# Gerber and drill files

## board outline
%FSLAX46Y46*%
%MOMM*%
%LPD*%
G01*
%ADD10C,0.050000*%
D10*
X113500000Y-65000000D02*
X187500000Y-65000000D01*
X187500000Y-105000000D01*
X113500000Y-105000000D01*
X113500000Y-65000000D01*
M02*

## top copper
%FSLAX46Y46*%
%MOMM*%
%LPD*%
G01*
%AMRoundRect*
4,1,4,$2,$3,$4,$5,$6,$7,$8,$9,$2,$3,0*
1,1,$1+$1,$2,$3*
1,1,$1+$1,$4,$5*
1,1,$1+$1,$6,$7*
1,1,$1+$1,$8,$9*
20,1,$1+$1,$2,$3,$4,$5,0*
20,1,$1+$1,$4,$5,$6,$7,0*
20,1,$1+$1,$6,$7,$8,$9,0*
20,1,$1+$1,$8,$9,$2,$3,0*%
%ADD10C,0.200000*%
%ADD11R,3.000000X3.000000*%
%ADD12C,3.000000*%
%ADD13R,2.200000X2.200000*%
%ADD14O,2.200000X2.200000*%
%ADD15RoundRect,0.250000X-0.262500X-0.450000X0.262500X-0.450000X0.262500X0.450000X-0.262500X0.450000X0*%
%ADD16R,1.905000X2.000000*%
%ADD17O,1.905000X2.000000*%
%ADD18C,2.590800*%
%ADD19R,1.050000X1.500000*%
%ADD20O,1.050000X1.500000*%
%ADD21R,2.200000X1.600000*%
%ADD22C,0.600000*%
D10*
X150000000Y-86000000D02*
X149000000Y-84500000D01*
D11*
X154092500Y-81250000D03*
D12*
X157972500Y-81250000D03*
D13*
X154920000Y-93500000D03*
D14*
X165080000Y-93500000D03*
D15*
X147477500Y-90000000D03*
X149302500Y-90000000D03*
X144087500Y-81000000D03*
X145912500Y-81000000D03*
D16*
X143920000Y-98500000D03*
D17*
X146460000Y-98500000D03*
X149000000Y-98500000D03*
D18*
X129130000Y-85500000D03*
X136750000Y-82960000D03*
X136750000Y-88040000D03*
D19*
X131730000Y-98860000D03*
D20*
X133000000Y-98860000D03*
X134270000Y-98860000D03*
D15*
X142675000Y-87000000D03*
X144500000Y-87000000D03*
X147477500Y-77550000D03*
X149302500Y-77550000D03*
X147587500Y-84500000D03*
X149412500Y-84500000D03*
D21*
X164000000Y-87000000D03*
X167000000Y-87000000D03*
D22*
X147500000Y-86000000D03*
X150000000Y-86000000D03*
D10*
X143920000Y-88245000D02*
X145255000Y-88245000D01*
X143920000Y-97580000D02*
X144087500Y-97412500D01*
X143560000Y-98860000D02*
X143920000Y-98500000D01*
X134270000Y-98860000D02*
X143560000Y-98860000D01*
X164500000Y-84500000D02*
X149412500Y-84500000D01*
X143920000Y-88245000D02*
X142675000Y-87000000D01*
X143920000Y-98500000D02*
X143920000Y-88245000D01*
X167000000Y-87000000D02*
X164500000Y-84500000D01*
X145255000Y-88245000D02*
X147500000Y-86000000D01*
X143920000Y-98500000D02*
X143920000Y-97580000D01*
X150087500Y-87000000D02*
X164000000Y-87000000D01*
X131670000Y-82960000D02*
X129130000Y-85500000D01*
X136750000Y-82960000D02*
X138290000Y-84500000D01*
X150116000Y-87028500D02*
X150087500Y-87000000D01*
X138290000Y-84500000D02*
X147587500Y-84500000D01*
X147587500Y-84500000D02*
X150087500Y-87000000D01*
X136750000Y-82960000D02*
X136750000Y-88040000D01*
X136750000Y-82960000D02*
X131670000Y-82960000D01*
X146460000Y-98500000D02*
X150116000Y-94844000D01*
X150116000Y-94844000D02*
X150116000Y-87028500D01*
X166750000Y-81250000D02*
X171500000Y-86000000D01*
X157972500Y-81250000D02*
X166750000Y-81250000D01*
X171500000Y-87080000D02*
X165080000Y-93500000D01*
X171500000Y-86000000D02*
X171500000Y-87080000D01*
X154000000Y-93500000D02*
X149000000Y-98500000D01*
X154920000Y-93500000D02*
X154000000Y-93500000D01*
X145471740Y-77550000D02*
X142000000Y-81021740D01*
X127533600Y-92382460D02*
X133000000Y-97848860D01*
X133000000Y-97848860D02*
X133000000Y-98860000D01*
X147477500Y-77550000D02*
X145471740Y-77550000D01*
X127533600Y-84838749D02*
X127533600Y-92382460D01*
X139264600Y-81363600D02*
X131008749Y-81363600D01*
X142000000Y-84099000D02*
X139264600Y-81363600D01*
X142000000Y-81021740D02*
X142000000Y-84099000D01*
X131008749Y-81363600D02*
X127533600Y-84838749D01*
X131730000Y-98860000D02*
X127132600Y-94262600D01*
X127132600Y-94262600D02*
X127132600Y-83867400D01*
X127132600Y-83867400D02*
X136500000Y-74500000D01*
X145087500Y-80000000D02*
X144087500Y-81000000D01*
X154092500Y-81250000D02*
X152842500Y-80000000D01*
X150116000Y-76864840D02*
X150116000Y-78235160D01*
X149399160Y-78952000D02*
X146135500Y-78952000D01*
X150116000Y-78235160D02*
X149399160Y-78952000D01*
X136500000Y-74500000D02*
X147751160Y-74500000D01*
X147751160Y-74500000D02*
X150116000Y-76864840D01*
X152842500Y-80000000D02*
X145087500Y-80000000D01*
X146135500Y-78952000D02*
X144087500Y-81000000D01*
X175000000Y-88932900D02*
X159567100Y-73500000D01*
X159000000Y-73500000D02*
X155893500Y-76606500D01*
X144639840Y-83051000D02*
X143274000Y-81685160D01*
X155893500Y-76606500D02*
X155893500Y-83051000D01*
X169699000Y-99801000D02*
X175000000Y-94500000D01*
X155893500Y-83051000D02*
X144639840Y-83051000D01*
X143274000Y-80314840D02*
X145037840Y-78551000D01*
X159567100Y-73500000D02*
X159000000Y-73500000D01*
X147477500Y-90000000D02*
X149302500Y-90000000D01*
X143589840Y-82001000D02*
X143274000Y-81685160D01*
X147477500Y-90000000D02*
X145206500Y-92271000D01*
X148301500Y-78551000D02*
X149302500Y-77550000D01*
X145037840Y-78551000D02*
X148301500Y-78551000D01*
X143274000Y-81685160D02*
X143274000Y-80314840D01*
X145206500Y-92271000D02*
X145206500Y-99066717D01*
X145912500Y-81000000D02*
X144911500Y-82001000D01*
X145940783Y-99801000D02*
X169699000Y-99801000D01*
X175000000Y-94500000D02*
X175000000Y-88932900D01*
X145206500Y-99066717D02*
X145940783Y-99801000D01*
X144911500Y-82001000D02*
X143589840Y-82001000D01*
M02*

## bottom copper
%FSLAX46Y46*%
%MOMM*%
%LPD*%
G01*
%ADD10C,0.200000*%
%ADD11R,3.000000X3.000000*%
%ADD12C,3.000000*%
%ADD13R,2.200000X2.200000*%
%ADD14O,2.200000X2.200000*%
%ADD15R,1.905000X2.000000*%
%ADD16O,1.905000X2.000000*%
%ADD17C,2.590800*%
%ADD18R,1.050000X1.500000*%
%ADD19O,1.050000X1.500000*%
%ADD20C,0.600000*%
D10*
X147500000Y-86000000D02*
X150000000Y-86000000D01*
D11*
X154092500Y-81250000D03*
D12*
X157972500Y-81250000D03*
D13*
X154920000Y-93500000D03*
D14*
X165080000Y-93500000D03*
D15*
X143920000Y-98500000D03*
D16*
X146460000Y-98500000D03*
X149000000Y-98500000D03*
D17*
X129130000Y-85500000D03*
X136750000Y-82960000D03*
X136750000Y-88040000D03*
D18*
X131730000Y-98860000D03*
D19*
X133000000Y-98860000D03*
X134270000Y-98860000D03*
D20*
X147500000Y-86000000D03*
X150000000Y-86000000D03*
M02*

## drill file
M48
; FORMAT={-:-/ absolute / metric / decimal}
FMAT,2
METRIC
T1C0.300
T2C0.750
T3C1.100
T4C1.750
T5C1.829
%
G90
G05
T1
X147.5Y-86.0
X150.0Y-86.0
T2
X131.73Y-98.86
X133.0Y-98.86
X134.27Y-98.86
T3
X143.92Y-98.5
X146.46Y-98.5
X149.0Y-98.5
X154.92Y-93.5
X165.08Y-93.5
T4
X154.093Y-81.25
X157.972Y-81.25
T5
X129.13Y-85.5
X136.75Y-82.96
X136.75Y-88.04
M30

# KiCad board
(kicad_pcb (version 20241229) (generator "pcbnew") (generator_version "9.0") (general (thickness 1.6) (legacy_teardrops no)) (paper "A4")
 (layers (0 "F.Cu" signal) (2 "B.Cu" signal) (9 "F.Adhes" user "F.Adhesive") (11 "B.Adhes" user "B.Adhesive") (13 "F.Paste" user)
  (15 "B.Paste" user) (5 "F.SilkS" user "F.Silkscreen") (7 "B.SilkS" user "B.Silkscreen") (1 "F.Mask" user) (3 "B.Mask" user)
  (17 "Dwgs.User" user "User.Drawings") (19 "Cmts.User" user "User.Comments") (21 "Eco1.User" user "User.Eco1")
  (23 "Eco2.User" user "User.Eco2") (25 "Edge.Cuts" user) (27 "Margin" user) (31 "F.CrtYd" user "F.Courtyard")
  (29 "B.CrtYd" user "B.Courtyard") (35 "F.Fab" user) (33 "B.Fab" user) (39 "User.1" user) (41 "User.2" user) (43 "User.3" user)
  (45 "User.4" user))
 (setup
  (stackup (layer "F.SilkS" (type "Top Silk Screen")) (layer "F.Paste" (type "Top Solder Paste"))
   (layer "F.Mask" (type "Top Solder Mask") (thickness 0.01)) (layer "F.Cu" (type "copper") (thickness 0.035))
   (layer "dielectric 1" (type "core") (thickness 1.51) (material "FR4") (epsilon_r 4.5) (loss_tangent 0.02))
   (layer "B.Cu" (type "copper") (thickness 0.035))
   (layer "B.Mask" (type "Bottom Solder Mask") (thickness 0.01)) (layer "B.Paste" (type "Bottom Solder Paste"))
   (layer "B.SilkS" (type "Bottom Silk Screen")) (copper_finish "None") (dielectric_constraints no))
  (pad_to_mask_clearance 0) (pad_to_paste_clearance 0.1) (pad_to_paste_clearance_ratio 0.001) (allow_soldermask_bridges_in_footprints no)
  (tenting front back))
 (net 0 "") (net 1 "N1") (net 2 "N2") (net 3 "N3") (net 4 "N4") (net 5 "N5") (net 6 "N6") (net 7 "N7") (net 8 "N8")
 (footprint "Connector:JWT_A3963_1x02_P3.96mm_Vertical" (layer "F.Cu") (at 154.0925 81.25)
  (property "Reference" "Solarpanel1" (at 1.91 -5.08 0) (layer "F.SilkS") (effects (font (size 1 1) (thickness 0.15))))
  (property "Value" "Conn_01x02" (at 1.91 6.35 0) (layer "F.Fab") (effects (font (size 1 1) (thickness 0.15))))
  (pad "1" thru_hole rect (at 0 0) (size 3 3) (drill 1.75) (layers "*.Cu" "*.Mask") (remove_unused_layers no) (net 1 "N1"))
  (pad "2" thru_hole circle (at 3.88 0) (size 3 3) (drill 1.75) (layers "*.Cu" "*.Mask") (remove_unused_layers no) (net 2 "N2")))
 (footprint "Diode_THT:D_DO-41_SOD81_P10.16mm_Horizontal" (layer "F.Cu") (at 154.92 93.5)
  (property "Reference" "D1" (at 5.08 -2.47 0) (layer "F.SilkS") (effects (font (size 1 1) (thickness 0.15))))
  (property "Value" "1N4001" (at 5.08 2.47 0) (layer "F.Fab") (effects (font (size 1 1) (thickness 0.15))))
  (pad "1" thru_hole rect (at 0 0) (size 2.2 2.2) (drill 1.1) (layers "*.Cu" "*.Mask") (remove_unused_layers no) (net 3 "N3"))
  (pad "2" thru_hole oval (at 10.16 0) (size 2.2 2.2) (drill 1.1) (layers "*.Cu" "*.Mask") (remove_unused_layers no) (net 2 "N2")))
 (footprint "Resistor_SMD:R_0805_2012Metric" (layer "F.Cu") (at 148.39 90)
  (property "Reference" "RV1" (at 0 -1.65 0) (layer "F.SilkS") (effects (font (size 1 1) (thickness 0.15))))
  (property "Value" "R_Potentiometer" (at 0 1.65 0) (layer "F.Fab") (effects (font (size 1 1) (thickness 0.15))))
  (pad "1" smd roundrect (at -0.9125 0) (size 1.025 1.4) (layers "F.Cu" "F.Mask" "F.Paste") (roundrect_rratio 0.243902) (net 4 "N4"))
  (pad "2" smd roundrect (at 0.9125 0) (size 1.025 1.4) (layers "F.Cu" "F.Mask" "F.Paste") (roundrect_rratio 0.243902) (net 4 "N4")))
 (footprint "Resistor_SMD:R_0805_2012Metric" (layer "F.Cu") (at 145 81)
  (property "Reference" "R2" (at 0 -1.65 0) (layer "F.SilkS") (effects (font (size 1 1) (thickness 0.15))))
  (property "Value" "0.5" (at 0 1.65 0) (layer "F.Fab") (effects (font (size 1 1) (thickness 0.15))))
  (pad "1" smd roundrect (at -0.9125 0) (size 1.025 1.4) (layers "F.Cu" "F.Mask" "F.Paste") (roundrect_rratio 0.243902) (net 1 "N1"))
  (pad "2" smd roundrect (at 0.9125 0) (size 1.025 1.4) (layers "F.Cu" "F.Mask" "F.Paste") (roundrect_rratio 0.243902) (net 4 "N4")))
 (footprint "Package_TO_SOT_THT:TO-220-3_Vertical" (layer "F.Cu") (at 143.92 98.5)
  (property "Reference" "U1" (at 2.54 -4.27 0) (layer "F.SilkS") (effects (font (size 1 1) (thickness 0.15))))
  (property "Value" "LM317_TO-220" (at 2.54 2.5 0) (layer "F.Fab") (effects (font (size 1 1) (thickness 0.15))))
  (pad "1" thru_hole rect (at 0 0) (size 1.905 2) (drill 1.1) (layers "*.Cu" "*.Mask") (remove_unused_layers no) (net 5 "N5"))
  (pad "2" thru_hole oval (at 2.54 0) (size 1.905 2) (drill 1.1) (layers "*.Cu" "*.Mask") (remove_unused_layers no) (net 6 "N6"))
  (pad "3" thru_hole oval (at 5.08 0) (size 1.905 2) (drill 1.1) (layers "*.Cu" "*.Mask") (remove_unused_layers no) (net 3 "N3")))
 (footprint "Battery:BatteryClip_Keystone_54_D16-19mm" (layer "F.Cu") (at 129.13 85.5)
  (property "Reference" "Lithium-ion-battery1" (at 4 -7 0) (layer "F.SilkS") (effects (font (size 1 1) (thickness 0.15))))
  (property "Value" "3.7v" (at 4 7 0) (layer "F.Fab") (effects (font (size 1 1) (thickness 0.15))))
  (pad "1" thru_hole circle (at 0 0 180) (size 2.5908 2.5908) (drill 1.8288) (layers "*.Cu" "*.Mask") (remove_unused_layers no) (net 6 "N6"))
  (pad "1" thru_hole circle (at 7.62 -2.54 180) (size 2.5908 2.5908) (drill 1.8288) (layers "*.Cu" "*.Mask") (remove_unused_layers no)
   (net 6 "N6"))
  (pad "1" thru_hole circle (at 7.62 2.54 180) (size 2.5908 2.5908) (drill 1.8288) (layers "*.Cu" "*.Mask") (remove_unused_layers no)
   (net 6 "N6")))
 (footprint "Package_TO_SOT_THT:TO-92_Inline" (layer "F.Cu") (at 131.73 98.86)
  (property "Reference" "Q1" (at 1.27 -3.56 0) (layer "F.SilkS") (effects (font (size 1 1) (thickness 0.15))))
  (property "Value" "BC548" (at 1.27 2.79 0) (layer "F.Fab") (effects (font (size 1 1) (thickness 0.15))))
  (pad "1" thru_hole rect (at 0 0) (size 1.05 1.5) (drill 0.75) (layers "*.Cu" "*.Mask") (remove_unused_layers no) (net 1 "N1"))
  (pad "2" thru_hole oval (at 1.27 0) (size 1.05 1.5) (drill 0.75) (layers "*.Cu" "*.Mask") (remove_unused_layers no) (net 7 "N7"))
  (pad "3" thru_hole oval (at 2.54 0) (size 1.05 1.5) (drill 0.75) (layers "*.Cu" "*.Mask") (remove_unused_layers no) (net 5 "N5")))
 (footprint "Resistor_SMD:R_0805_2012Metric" (layer "F.Cu") (at 143.5875 87)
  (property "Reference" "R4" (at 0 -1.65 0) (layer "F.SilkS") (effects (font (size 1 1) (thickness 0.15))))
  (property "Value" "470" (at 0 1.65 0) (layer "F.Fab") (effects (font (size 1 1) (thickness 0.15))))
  (pad "1" smd roundrect (at -0.9125 0) (size 1.025 1.4) (layers "F.Cu" "F.Mask" "F.Paste") (roundrect_rratio 0.243902) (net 5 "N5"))
  (pad "2" smd roundrect (at 0.9125 0) (size 1.025 1.4) (layers "F.Cu" "F.Mask" "F.Paste") (roundrect_rratio 0.243902) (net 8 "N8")))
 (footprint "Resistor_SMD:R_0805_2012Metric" (layer "F.Cu") (at 148.39 77.55)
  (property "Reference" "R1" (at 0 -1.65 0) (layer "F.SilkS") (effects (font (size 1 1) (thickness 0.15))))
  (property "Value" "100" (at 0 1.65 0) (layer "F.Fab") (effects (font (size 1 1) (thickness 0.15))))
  (pad "1" smd roundrect (at -0.9125 0) (size 1.025 1.4) (layers "F.Cu" "F.Mask" "F.Paste") (roundrect_rratio 0.243902) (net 7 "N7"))
  (pad "2" smd roundrect (at 0.9125 0) (size 1.025 1.4) (layers "F.Cu" "F.Mask" "F.Paste") (roundrect_rratio 0.243902) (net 4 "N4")))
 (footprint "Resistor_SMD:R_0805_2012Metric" (layer "F.Cu") (at 148.5 84.5)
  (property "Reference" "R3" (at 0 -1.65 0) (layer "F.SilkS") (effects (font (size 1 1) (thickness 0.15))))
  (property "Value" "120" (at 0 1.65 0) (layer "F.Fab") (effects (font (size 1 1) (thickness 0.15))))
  (pad "1" smd roundrect (at -0.9125 0) (size 1.025 1.4) (layers "F.Cu" "F.Mask" "F.Paste") (roundrect_rratio 0.243902) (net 6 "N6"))
  (pad "2" smd roundrect (at 0.9125 0) (size 1.025 1.4) (layers "F.Cu" "F.Mask" "F.Paste") (roundrect_rratio 0.243902) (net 5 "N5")))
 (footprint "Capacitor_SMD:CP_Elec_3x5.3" (layer "F.Cu") (at 165.5 87)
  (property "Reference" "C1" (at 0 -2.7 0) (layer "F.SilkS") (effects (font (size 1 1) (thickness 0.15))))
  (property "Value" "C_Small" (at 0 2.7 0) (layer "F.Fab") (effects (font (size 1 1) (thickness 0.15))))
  (pad "1" smd rect (at -1.5 0) (size 2.2 1.6) (layers "F.Cu" "F.Mask" "F.Paste") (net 6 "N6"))
  (pad "2" smd rect (at 1.5 0) (size 2.2 1.6) (layers "F.Cu" "F.Mask" "F.Paste") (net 5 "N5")))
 (gr_line (start 150 86) (end 149 84.5) (stroke (width 0.2) (type default)) (layer "F.Cu") (net 5))
 (gr_line (start 147.5 86) (end 150 86) (stroke (width 0.2) (type default)) (layer "B.Cu") (net 5))
 (gr_rect (start 113.5 65) (end 187.5 105) (stroke (width 0.05) (type default)) (fill no) (layer "Edge.Cuts"))
 (segment (start 143.92 88.245) (end 145.255 88.245) (width 0.2) (layer "F.Cu") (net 5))
 (segment (start 143.92 97.58) (end 144.0875 97.4125) (width 0.2) (layer "F.Cu") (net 5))
 (segment (start 143.56 98.86) (end 143.92 98.5) (width 0.2) (layer "F.Cu") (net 5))
 (segment (start 134.27 98.86) (end 143.56 98.86) (width 0.2) (layer "F.Cu") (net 5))
 (segment (start 164.5 84.5) (end 149.4125 84.5) (width 0.2) (layer "F.Cu") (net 5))
 (segment (start 143.92 88.245) (end 142.675 87) (width 0.2) (layer "F.Cu") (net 5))
 (segment (start 143.92 98.5) (end 143.92 88.245) (width 0.2) (layer "F.Cu") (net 5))
 (segment (start 167 87) (end 164.5 84.5) (width 0.2) (layer "F.Cu") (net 5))
 (segment (start 145.255 88.245) (end 147.5 86) (width 0.2) (layer "F.Cu") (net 5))
 (segment (start 143.92 98.5) (end 143.92 97.58) (width 0.2) (layer "F.Cu") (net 5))
 (via (at 147.5 86) (size 0.6) (drill 0.3) (layers "F.Cu" "B.Cu") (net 5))
 (via (at 150 86) (size 0.6) (drill 0.3) (layers "F.Cu" "B.Cu") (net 5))
 (segment (start 150.0875 87) (end 164 87) (width 0.2) (layer "F.Cu") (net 6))
 (segment (start 131.67 82.96) (end 129.13 85.5) (width 0.2) (layer "F.Cu") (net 6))
 (segment (start 136.75 82.96) (end 138.29 84.5) (width 0.2) (layer "F.Cu") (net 6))
 (segment (start 150.116 87.0285) (end 150.0875 87) (width 0.2) (layer "F.Cu") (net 6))
 (segment (start 138.29 84.5) (end 147.5875 84.5) (width 0.2) (layer "F.Cu") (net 6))
 (segment (start 147.5875 84.5) (end 150.0875 87) (width 0.2) (layer "F.Cu") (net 6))
 (segment (start 136.75 82.96) (end 136.75 88.04) (width 0.2) (layer "F.Cu") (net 6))
 (segment (start 136.75 82.96) (end 131.67 82.96) (width 0.2) (layer "F.Cu") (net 6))
 (segment (start 146.46 98.5) (end 150.116 94.844) (width 0.2) (layer "F.Cu") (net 6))
 (segment (start 150.116 94.844) (end 150.116 87.0285) (width 0.2) (layer "F.Cu") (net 6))
 (segment (start 166.75 81.25) (end 171.5 86) (width 0.2) (layer "F.Cu") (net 2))
 (segment (start 157.9725 81.25) (end 166.75 81.25) (width 0.2) (layer "F.Cu") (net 2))
 (segment (start 171.5 87.08) (end 165.08 93.5) (width 0.2) (layer "F.Cu") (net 2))
 (segment (start 171.5 86) (end 171.5 87.08) (width 0.2) (layer "F.Cu") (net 2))
 (segment (start 154 93.5) (end 149 98.5) (width 0.2) (layer "F.Cu") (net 3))
 (segment (start 154.92 93.5) (end 154 93.5) (width 0.2) (layer "F.Cu") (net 3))
 (segment (start 145.47174 77.55) (end 142 81.02174) (width 0.2) (layer "F.Cu") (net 7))
 (segment (start 127.5336 92.38246) (end 133 97.84886) (width 0.2) (layer "F.Cu") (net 7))
 (segment (start 133 97.84886) (end 133 98.86) (width 0.2) (layer "F.Cu") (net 7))
 (segment (start 147.4775 77.55) (end 145.47174 77.55) (width 0.2) (layer "F.Cu") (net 7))
 (segment (start 127.5336 84.838749) (end 127.5336 92.38246) (width 0.2) (layer "F.Cu") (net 7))
 (segment (start 139.2646 81.3636) (end 131.008749 81.3636) (width 0.2) (layer "F.Cu") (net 7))
 (segment (start 142 84.099) (end 139.2646 81.3636) (width 0.2) (layer "F.Cu") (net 7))
 (segment (start 142 81.02174) (end 142 84.099) (width 0.2) (layer "F.Cu") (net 7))
 (segment (start 131.008749 81.3636) (end 127.5336 84.838749) (width 0.2) (layer "F.Cu") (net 7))
 (segment (start 131.73 98.86) (end 127.1326 94.2626) (width 0.2) (layer "F.Cu") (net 1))
 (segment (start 127.1326 94.2626) (end 127.1326 83.8674) (width 0.2) (layer "F.Cu") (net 1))
 (segment (start 127.1326 83.8674) (end 136.5 74.5) (width 0.2) (layer "F.Cu") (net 1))
 (segment (start 145.0875 80) (end 144.0875 81) (width 0.2) (layer "F.Cu") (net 1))
 (segment (start 154.0925 81.25) (end 152.8425 80) (width 0.2) (layer "F.Cu") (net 1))
 (segment (start 150.116 76.86484) (end 150.116 78.23516) (width 0.2) (layer "F.Cu") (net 1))
 (segment (start 149.39916 78.952) (end 146.1355 78.952) (width 0.2) (layer "F.Cu") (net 1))
 (segment (start 150.116 78.23516) (end 149.39916 78.952) (width 0.2) (layer "F.Cu") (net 1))
 (segment (start 136.5 74.5) (end 147.75116 74.5) (width 0.2) (layer "F.Cu") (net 1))
 (segment (start 147.75116 74.5) (end 150.116 76.86484) (width 0.2) (layer "F.Cu") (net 1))
 (segment (start 152.8425 80) (end 145.0875 80) (width 0.2) (layer "F.Cu") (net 1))
 (segment (start 146.1355 78.952) (end 144.0875 81) (width 0.2) (layer "F.Cu") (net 1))
 (segment (start 175 88.9329) (end 159.5671 73.5) (width 0.2) (layer "F.Cu") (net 4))
 (segment (start 159 73.5) (end 155.8935 76.6065) (width 0.2) (layer "F.Cu") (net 4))
 (segment (start 144.63984 83.051) (end 143.274 81.68516) (width 0.2) (layer "F.Cu") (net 4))
 (segment (start 155.8935 76.6065) (end 155.8935 83.051) (width 0.2) (layer "F.Cu") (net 4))
 (segment (start 169.699 99.801) (end 175 94.5) (width 0.2) (layer "F.Cu") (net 4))
 (segment (start 155.8935 83.051) (end 144.63984 83.051) (width 0.2) (layer "F.Cu") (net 4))
 (segment (start 143.274 80.31484) (end 145.03784 78.551) (width 0.2) (layer "F.Cu") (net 4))
 (segment (start 159.5671 73.5) (end 159 73.5) (width 0.2) (layer "F.Cu") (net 4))
 (segment (start 147.4775 90) (end 149.3025 90) (width 0.2) (layer "F.Cu") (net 4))
 (segment (start 143.58984 82.001) (end 143.274 81.68516) (width 0.2) (layer "F.Cu") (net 4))
 (segment (start 147.4775 90) (end 145.2065 92.271) (width 0.2) (layer "F.Cu") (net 4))
 (segment (start 148.3015 78.551) (end 149.3025 77.55) (width 0.2) (layer "F.Cu") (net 4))
 (segment (start 145.03784 78.551) (end 148.3015 78.551) (width 0.2) (layer "F.Cu") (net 4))
 (segment (start 143.274 81.68516) (end 143.274 80.31484) (width 0.2) (layer "F.Cu") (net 4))
 (segment (start 145.2065 92.271) (end 145.2065 99.066717) (width 0.2) (layer "F.Cu") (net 4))
 (segment (start 145.9125 81) (end 144.9115 82.001) (width 0.2) (layer "F.Cu") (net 4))
 (segment (start 145.940783 99.801) (end 169.699 99.801) (width 0.2) (layer "F.Cu") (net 4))
 (segment (start 175 94.5) (end 175 88.9329) (width 0.2) (layer "F.Cu") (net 4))
 (segment (start 145.2065 99.066717) (end 145.940783 99.801) (width 0.2) (layer "F.Cu") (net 4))
 (segment (start 144.9115 82.001) (end 143.58984 82.001) (width 0.2) (layer "F.Cu") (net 4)))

